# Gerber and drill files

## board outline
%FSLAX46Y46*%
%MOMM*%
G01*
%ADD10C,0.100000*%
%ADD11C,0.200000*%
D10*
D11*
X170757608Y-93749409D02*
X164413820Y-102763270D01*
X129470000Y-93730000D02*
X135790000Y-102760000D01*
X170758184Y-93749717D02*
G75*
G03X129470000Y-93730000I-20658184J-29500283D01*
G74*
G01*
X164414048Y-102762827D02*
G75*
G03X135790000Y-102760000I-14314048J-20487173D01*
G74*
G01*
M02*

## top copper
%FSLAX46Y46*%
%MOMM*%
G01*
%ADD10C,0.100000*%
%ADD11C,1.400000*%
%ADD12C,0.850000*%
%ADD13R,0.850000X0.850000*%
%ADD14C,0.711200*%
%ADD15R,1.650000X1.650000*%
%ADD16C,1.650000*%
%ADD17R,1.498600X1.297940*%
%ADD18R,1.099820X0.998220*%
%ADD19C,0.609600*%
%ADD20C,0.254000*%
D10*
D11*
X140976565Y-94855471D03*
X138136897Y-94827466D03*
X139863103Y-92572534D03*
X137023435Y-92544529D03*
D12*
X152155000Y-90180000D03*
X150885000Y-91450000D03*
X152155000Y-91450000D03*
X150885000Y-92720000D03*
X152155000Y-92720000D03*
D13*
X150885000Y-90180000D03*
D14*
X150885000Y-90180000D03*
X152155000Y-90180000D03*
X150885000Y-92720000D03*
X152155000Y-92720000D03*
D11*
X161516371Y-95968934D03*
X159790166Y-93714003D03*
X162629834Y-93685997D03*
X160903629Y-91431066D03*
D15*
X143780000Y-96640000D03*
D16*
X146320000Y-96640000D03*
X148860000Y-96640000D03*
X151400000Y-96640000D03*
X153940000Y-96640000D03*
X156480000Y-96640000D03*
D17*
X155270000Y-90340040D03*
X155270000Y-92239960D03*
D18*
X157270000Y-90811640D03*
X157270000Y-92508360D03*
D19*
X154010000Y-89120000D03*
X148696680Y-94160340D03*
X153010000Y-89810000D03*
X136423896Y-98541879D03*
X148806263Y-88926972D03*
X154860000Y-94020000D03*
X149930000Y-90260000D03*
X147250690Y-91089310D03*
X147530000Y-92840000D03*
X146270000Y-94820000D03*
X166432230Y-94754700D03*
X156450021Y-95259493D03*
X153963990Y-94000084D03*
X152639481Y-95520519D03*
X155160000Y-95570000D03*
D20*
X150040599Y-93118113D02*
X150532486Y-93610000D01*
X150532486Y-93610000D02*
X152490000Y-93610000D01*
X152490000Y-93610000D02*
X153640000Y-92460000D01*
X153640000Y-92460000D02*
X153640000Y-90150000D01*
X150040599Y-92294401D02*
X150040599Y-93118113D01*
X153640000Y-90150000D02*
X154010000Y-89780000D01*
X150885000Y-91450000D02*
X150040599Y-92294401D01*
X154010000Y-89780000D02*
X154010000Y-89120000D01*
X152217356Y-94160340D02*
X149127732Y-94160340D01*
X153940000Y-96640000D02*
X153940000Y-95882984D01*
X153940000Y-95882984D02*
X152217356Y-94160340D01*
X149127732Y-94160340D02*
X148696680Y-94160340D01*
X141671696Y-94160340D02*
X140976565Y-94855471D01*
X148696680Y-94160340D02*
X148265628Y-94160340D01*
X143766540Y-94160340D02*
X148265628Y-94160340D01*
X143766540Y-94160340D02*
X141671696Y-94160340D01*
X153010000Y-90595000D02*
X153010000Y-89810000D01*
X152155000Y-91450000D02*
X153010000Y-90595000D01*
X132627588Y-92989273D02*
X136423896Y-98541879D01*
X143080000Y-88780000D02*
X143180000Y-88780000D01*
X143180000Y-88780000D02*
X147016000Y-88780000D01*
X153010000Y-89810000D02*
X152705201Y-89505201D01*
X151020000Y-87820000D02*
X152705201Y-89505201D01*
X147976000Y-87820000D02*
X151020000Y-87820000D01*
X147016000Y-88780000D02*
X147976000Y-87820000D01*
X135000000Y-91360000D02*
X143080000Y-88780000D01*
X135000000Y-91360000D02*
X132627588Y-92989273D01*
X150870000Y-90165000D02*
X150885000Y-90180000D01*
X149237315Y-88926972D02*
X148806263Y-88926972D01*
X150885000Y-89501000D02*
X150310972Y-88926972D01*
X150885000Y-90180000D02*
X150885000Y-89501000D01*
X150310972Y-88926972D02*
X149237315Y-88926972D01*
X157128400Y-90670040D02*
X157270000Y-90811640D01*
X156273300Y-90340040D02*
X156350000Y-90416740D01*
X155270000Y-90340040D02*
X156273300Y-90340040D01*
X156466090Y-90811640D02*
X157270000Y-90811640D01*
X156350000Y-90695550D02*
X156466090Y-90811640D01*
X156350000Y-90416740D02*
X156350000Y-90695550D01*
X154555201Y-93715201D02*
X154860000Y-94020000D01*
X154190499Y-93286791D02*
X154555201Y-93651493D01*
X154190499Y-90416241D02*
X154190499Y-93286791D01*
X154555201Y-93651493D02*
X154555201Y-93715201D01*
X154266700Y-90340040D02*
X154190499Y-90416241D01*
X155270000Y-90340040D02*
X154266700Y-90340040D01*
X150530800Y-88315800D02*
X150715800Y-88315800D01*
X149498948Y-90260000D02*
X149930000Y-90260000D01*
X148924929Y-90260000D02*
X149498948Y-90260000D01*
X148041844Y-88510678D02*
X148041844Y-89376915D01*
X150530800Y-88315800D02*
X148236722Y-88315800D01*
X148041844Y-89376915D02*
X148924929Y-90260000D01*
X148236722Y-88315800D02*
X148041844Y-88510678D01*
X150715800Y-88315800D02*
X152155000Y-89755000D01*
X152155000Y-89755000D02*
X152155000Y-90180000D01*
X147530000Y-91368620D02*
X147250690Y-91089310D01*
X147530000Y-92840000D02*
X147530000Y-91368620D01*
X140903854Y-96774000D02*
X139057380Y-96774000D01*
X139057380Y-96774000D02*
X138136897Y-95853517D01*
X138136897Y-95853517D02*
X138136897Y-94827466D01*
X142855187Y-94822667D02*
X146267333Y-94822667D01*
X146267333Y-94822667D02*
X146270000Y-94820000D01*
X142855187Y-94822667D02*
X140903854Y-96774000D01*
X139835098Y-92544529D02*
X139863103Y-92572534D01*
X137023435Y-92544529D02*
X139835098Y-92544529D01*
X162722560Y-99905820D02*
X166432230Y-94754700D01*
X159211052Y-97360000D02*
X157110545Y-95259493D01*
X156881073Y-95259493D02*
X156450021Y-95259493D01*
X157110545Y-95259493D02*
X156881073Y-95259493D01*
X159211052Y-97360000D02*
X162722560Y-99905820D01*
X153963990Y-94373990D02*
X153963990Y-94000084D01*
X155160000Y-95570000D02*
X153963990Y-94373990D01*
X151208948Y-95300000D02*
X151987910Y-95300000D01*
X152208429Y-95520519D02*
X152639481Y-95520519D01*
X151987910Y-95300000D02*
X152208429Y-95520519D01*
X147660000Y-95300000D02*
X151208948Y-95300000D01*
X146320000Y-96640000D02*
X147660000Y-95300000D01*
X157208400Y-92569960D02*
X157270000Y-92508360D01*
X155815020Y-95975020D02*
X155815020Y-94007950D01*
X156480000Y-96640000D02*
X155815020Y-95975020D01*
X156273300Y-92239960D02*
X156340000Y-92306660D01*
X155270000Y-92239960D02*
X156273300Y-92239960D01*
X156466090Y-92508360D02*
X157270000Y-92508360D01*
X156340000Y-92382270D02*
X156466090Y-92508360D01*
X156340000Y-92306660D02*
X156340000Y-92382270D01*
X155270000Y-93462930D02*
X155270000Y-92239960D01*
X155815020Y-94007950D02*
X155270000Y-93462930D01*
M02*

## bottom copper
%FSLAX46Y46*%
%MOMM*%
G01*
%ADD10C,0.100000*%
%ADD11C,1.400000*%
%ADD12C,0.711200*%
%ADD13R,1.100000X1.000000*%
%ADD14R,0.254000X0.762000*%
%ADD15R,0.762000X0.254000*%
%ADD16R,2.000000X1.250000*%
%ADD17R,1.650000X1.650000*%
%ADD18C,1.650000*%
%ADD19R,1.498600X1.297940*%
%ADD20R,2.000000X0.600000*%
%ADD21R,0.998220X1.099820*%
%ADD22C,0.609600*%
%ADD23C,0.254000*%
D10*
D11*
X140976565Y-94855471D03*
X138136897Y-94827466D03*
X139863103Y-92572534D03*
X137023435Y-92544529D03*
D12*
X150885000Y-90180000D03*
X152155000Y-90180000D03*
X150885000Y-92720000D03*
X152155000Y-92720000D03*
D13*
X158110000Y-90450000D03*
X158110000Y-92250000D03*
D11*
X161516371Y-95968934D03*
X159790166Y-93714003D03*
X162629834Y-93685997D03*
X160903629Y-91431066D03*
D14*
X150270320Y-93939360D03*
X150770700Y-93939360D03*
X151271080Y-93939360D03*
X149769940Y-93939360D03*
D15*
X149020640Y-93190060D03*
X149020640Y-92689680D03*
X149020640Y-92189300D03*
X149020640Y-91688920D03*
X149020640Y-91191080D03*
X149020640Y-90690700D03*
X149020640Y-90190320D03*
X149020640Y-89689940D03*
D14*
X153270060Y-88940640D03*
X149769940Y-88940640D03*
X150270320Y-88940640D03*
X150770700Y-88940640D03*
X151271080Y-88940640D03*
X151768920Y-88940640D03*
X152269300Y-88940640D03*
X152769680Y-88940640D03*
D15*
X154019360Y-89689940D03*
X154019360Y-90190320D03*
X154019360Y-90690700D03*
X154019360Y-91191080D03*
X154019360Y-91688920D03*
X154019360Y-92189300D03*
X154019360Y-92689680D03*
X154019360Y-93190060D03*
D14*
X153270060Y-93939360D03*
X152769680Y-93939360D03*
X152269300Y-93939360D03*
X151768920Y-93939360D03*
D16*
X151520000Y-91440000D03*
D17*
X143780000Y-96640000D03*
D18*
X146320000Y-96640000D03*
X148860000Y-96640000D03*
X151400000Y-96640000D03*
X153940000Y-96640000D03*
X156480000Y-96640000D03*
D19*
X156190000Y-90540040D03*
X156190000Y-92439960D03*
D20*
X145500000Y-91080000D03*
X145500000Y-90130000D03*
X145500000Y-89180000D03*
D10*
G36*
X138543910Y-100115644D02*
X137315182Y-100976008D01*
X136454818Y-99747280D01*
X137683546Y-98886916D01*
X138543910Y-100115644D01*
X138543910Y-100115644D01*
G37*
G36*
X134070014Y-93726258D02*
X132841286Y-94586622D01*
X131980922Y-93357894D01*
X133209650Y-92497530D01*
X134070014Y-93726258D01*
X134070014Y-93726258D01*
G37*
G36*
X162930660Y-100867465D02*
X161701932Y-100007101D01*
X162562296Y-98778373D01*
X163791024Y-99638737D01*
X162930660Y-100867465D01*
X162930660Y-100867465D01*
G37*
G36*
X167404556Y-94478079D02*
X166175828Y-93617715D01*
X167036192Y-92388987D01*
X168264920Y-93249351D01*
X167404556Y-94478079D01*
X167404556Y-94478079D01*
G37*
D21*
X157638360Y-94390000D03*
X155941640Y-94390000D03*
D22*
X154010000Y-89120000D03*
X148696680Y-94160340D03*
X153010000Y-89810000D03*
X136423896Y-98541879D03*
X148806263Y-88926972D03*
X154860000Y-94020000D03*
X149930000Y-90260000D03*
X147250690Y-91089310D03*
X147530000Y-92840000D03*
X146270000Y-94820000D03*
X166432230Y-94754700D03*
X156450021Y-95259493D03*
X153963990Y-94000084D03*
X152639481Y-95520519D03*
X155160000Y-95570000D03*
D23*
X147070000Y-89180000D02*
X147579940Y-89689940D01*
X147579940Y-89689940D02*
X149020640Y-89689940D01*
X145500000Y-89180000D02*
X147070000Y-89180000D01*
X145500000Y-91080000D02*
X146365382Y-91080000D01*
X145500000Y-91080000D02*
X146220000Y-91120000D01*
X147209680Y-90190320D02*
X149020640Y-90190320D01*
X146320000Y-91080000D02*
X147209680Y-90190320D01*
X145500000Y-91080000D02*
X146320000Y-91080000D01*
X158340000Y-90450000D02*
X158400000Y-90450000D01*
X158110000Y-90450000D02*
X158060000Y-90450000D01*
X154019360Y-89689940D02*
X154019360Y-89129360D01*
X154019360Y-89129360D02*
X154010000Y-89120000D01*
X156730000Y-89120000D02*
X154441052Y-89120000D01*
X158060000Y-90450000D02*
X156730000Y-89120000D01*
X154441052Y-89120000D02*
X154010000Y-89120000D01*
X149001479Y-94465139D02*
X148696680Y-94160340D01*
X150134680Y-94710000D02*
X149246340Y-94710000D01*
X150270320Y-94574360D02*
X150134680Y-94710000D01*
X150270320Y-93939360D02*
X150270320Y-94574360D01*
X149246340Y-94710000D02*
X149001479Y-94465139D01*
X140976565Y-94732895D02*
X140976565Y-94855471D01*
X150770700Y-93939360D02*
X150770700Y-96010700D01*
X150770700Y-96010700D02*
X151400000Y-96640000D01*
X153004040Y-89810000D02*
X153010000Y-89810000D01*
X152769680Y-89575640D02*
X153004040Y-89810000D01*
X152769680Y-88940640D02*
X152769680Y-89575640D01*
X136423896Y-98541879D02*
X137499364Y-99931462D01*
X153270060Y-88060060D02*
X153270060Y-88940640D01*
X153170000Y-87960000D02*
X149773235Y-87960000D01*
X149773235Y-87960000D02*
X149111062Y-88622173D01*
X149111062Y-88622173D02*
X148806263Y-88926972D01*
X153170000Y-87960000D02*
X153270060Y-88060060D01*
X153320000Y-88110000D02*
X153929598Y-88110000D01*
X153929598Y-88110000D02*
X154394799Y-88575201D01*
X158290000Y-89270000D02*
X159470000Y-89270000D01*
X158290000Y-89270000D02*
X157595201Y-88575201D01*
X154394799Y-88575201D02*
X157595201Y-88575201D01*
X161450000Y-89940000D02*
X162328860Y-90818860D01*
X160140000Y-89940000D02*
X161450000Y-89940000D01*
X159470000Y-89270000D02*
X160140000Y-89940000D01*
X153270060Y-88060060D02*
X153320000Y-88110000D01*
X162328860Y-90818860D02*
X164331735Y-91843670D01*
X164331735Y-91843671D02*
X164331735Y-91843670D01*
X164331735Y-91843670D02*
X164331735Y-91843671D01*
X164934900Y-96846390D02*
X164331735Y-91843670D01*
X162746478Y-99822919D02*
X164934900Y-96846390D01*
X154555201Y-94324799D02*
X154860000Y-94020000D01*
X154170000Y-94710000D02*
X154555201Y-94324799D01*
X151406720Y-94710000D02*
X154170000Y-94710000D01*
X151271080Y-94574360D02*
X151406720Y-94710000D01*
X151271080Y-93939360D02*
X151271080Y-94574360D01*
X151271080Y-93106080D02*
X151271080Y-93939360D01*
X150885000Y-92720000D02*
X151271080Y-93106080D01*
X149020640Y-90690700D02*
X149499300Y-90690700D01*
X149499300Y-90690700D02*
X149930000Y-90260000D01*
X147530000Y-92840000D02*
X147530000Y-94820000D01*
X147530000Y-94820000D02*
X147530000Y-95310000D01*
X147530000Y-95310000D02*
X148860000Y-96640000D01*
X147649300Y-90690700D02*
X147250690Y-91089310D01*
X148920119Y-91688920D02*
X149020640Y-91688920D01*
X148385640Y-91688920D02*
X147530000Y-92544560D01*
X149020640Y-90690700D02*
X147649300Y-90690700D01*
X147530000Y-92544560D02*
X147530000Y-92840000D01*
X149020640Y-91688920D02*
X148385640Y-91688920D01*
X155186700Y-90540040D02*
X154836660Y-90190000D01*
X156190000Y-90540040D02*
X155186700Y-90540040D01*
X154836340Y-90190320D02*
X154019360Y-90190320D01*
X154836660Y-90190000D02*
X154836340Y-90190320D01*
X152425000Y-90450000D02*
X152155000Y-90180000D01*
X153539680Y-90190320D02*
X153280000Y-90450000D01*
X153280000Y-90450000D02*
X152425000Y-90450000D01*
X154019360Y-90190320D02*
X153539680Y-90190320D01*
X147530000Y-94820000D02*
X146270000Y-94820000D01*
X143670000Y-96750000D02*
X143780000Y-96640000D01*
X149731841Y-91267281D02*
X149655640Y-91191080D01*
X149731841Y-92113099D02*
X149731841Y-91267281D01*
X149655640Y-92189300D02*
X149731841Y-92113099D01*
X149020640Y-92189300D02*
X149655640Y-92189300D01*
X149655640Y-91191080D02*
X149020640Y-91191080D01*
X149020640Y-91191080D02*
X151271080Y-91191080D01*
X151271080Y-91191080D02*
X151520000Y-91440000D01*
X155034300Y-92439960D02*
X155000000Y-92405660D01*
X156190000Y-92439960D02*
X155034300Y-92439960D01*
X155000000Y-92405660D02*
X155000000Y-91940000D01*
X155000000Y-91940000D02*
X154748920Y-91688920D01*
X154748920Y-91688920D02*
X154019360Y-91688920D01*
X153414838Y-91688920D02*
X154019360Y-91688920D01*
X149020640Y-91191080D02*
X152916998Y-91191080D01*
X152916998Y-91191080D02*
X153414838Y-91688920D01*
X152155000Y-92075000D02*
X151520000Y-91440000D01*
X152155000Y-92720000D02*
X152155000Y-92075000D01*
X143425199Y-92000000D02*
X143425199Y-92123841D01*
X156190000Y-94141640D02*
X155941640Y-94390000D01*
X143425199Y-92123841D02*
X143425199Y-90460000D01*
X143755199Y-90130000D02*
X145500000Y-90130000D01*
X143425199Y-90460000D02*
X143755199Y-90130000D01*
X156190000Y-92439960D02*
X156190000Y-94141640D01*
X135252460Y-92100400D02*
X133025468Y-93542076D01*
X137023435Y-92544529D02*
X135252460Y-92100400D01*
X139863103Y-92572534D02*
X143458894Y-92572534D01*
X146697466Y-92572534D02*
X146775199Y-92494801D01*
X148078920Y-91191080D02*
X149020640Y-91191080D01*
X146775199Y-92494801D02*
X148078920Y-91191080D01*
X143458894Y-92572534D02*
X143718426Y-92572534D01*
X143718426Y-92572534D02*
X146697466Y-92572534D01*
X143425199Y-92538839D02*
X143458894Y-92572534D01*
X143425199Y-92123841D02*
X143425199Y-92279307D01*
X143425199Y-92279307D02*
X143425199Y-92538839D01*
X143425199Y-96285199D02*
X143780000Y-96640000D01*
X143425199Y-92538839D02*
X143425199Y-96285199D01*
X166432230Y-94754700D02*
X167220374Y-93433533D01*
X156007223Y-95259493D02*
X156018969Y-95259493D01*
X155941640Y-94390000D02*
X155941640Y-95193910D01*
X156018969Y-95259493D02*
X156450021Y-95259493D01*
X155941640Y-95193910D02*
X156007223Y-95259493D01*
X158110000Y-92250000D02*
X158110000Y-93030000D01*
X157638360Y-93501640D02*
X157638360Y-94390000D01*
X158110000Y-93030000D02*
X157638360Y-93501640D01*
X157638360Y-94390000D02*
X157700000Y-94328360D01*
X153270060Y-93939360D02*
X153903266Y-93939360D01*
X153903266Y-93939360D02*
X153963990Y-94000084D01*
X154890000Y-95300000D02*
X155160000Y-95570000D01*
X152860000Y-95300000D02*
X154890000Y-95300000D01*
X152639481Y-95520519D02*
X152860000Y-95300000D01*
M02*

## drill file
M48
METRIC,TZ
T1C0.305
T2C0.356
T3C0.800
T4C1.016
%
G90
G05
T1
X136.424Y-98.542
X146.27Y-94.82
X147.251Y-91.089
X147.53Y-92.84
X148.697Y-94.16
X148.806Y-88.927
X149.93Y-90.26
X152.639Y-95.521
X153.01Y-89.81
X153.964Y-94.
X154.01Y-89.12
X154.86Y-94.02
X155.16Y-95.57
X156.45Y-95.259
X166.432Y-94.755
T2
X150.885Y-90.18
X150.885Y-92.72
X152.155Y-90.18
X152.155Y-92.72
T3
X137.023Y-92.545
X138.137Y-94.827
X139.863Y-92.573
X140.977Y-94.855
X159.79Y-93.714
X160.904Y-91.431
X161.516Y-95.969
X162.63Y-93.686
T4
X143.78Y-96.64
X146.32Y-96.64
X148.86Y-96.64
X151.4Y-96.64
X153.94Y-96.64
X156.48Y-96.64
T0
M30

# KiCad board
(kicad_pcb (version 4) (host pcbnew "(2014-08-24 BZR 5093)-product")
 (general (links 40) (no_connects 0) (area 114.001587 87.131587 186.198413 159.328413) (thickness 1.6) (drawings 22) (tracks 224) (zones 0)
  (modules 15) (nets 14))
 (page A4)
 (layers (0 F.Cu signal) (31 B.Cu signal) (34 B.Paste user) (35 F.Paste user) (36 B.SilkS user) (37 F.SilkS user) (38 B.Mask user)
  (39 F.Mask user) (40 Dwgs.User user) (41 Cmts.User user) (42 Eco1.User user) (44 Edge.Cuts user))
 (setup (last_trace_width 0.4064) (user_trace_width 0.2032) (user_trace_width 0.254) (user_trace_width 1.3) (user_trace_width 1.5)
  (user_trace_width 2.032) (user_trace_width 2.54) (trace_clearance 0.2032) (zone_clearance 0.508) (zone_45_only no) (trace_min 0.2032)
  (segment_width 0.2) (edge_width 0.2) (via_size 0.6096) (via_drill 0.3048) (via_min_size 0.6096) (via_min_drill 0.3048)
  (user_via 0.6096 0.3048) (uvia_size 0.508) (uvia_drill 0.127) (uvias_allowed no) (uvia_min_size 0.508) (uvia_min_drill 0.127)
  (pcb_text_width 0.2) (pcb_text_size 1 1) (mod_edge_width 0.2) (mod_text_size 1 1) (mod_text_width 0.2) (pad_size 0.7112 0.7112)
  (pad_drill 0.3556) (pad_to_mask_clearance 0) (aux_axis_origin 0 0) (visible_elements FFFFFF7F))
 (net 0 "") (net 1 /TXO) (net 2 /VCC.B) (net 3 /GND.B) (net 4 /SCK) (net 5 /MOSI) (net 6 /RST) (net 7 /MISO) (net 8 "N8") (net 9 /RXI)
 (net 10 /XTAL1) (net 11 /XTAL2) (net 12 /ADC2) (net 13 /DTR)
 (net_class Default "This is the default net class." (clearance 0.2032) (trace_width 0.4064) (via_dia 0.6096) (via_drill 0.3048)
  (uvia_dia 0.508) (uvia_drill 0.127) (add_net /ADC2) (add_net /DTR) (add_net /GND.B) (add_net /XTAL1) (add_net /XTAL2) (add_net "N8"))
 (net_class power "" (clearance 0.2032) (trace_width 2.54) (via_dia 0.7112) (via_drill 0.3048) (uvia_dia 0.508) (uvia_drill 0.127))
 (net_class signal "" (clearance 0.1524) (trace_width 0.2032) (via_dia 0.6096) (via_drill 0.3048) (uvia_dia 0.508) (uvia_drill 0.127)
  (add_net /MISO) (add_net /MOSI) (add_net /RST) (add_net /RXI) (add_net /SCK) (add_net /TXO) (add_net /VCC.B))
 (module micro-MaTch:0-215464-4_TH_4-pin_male (layer F.Cu) (at 139 93.7 296)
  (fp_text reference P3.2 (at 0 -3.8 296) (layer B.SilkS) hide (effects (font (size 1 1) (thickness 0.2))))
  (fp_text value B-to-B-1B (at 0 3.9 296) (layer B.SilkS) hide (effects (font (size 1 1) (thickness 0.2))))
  (pad 1 thru_hole circle (at 1.905 -1.27 296) (size 1.4 1.4) (drill 0.8) (layers *.Cu *.Mask) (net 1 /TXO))
  (pad 2 thru_hole circle (at 0.635 1.27 296) (size 1.4 1.4) (drill 0.8) (layers *.Cu *.Mask) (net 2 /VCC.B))
  (pad 3 thru_hole circle (at -0.635 -1.27 296) (size 1.4 1.4) (drill 0.8) (layers *.Cu *.Mask) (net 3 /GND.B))
  (pad 4 thru_hole circle (at -1.905 1.27 296) (size 1.4 1.4) (drill 0.8) (layers *.Cu *.Mask) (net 3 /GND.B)))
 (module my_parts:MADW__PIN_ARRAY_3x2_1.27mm (layer F.Cu) (at 151.52 91.45 270) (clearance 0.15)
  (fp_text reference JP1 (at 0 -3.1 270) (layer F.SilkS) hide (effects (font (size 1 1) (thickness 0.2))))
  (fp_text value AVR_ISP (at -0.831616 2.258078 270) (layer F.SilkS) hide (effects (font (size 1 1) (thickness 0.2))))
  (pad 2 smd circle (at -1.27 -0.635 270) (size 0.85 0.85) (layers F.Cu F.Mask) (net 2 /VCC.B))
  (pad 3 smd circle (at 0 0.635 270) (size 0.85 0.85) (layers F.Cu F.Mask) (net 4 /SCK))
  (pad 4 smd circle (at 0 -0.635 270) (size 0.85 0.85) (layers F.Cu F.Mask) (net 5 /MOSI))
  (pad 5 smd circle (at 1.27 0.635 270) (size 0.85 0.85) (layers F.Cu F.Mask) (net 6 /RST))
  (pad 6 smd circle (at 1.27 -0.635 270) (size 0.85 0.85) (layers F.Cu F.Mask) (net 3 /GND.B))
  (pad 1 smd rect (at -1.27 0.635 270) (size 0.85 0.85) (layers F.Cu F.Mask) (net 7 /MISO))
  (pad 1 thru_hole circle (at -1.27 0.635 270) (size 0.7112 0.7112) (drill 0.3556) (layers *.Cu F.Mask) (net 7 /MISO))
  (pad 2 thru_hole circle (at -1.27 -0.635 270) (size 0.7112 0.7112) (drill 0.3556) (layers *.Cu F.Mask) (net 2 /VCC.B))
  (pad 5 thru_hole circle (at 1.27 0.635 270) (size 0.7112 0.7112) (drill 0.3556) (layers *.Cu F.Mask) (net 6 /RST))
  (pad 6 thru_hole circle (at 1.27 -0.635 270) (size 0.7112 0.7112) (drill 0.3556) (layers *.Cu F.Mask) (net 3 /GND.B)))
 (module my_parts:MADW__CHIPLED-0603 (layer B.Cu) (at 158.11 91.35 270)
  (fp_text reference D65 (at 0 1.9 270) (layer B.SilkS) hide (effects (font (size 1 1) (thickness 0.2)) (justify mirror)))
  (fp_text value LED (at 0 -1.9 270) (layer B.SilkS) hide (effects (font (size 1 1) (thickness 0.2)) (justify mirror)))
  (pad 1 smd rect (at -0.9 0 270) (size 1 1.1) (layers B.Cu B.Paste B.Mask) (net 4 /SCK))
  (pad 2 smd rect (at 0.9 0 270) (size 1 1.1) (layers B.Cu B.Paste B.Mask) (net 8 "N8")))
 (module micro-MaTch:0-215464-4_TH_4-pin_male (layer F.Cu) (at 161.21 93.7 244)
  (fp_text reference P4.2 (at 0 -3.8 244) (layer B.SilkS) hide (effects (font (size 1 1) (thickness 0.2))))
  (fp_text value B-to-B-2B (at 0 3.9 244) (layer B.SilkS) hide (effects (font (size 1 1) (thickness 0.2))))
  (pad 1 thru_hole circle (at 1.905 -1.27 244) (size 1.4 1.4) (drill 0.8) (layers *.Cu *.Mask))
  (pad 2 thru_hole circle (at 0.635 1.27 244) (size 1.4 1.4) (drill 0.8) (layers *.Cu *.Mask))
  (pad 3 thru_hole circle (at -0.635 -1.27 244) (size 1.4 1.4) (drill 0.8) (layers *.Cu *.Mask))
  (pad 4 thru_hole circle (at -1.905 1.27 244) (size 1.4 1.4) (drill 0.8) (layers *.Cu *.Mask)))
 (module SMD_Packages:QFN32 (layer B.Cu) (at 151.52 91.44)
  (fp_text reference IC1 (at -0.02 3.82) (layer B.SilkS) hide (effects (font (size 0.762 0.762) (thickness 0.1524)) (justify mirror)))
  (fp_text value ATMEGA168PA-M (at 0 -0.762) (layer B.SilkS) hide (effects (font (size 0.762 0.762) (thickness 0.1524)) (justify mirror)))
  (pad 31 smd rect (at -1.24968 2.49936) (size 0.254 0.762) (layers B.Cu B.Paste B.Mask) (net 1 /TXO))
  (pad 30 smd rect (at -0.7493 2.49936) (size 0.254 0.762) (layers B.Cu B.Paste B.Mask) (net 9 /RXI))
  (pad 29 smd rect (at -0.24892 2.49936) (size 0.254 0.762) (layers B.Cu B.Paste B.Mask) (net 6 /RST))
  (pad 32 smd rect (at -1.75006 2.49936) (size 0.254 0.762) (layers B.Cu B.Paste B.Mask))
  (pad 1 smd rect (at -2.49936 1.75006 270) (size 0.254 0.762) (layers B.Cu B.Paste B.Mask))
  (pad 2 smd rect (at -2.49936 1.24968 270) (size 0.254 0.762) (layers B.Cu B.Paste B.Mask))
  (pad 3 smd rect (at -2.49936 0.7493 270) (size 0.254 0.762) (layers B.Cu B.Paste B.Mask) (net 3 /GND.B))
  (pad 4 smd rect (at -2.49936 0.24892 270) (size 0.254 0.762) (layers B.Cu B.Paste B.Mask) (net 2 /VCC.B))
  (pad 5 smd rect (at -2.49936 -0.24892 270) (size 0.254 0.762) (layers B.Cu B.Paste B.Mask) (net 3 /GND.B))
  (pad 6 smd rect (at -2.49936 -0.7493 270) (size 0.254 0.762) (layers B.Cu B.Paste B.Mask) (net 2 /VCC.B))
  (pad 7 smd rect (at -2.49936 -1.24968 270) (size 0.254 0.762) (layers B.Cu B.Paste B.Mask) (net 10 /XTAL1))
  (pad 8 smd rect (at -2.49936 -1.75006 270) (size 0.254 0.762) (layers B.Cu B.Paste B.Mask) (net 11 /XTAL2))
  (pad 16 smd rect (at 1.75006 -2.49936) (size 0.254 0.762) (layers B.Cu B.Paste B.Mask) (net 7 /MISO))
  (pad 9 smd rect (at -1.75006 -2.49936) (size 0.254 0.762) (layers B.Cu B.Paste B.Mask))
  (pad 10 smd rect (at -1.24968 -2.49936) (size 0.254 0.762) (layers B.Cu B.Paste B.Mask))
  (pad 11 smd rect (at -0.7493 -2.49936) (size 0.254 0.762) (layers B.Cu B.Paste B.Mask))
  (pad 12 smd rect (at -0.24892 -2.49936) (size 0.254 0.762) (layers B.Cu B.Paste B.Mask))
  (pad 13 smd rect (at 0.24892 -2.49936) (size 0.254 0.762) (layers B.Cu B.Paste B.Mask))
  (pad 14 smd rect (at 0.7493 -2.49936) (size 0.254 0.762) (layers B.Cu B.Paste B.Mask))
  (pad 15 smd rect (at 1.24968 -2.49936) (size 0.254 0.762) (layers B.Cu B.Paste B.Mask) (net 5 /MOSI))
  (pad 17 smd rect (at 2.49936 -1.75006 270) (size 0.254 0.762) (layers B.Cu B.Paste B.Mask) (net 4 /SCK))
  (pad 18 smd rect (at 2.49936 -1.24968 270) (size 0.254 0.762) (layers B.Cu B.Paste B.Mask) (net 2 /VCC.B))
  (pad 19 smd rect (at 2.49936 -0.7493 270) (size 0.254 0.762) (layers B.Cu B.Paste B.Mask))
  (pad 20 smd rect (at 2.49936 -0.24892 270) (size 0.254 0.762) (layers B.Cu B.Paste B.Mask))
  (pad 21 smd rect (at 2.49936 0.24892 270) (size 0.254 0.762) (layers B.Cu B.Paste B.Mask) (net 3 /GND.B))
  (pad 22 smd rect (at 2.49936 0.7493 270) (size 0.254 0.762) (layers B.Cu B.Paste B.Mask))
  (pad 23 smd rect (at 2.49936 1.24968 270) (size 0.254 0.762) (layers B.Cu B.Paste B.Mask))
  (pad 24 smd rect (at 2.49936 1.75006 270) (size 0.254 0.762) (layers B.Cu B.Paste B.Mask))
  (pad 25 smd rect (at 1.75006 2.49936) (size 0.254 0.762) (layers B.Cu B.Paste B.Mask) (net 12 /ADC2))
  (pad 26 smd rect (at 1.24968 2.49936) (size 0.254 0.762) (layers B.Cu B.Paste B.Mask))
  (pad 27 smd rect (at 0.7493 2.49936) (size 0.254 0.762) (layers B.Cu B.Paste B.Mask))
  (pad 28 smd rect (at 0.24892 2.49936) (size 0.254 0.762) (layers B.Cu B.Paste B.Mask))
  (pad 33 smd rect (at 0 0) (size 2 1.25) (layers B.Cu B.Paste B.Mask) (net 3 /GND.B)))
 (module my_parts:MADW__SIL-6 (layer B.Cu) (at 150.13 96.64)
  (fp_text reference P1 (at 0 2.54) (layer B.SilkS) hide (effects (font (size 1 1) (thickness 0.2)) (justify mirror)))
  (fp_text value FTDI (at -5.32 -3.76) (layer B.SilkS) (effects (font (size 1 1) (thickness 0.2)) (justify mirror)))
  (pad 1 thru_hole rect (at -6.35 0) (size 1.65 1.65) (drill 1.016) (layers *.Cu *.Mask B.SilkS) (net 3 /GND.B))
  (pad 2 thru_hole circle (at -3.81 0) (size 1.65 1.65) (drill 1.016) (layers *.Cu *.Mask B.SilkS) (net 12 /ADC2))
  (pad 3 thru_hole circle (at -1.27 0) (size 1.65 1.65) (drill 1.016) (layers *.Cu *.Mask B.SilkS) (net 2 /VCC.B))
  (pad 4 thru_hole circle (at 1.27 0) (size 1.65 1.65) (drill 1.016) (layers *.Cu *.Mask B.SilkS) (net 9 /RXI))
  (pad 5 thru_hole circle (at 3.81 0) (size 1.65 1.65) (drill 1.016) (layers *.Cu *.Mask B.SilkS) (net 1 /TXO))
  (pad 6 thru_hole circle (at 6.35 0) (size 1.65 1.65) (drill 1.016) (layers *.Cu *.Mask B.SilkS) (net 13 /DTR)))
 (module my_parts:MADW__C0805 (layer B.Cu) (at 156.19 91.49 270)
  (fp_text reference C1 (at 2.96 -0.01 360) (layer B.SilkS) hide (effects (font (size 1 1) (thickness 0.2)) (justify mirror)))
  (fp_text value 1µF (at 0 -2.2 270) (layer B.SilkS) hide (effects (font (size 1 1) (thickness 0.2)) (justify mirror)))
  (pad 1 smd rect (at -0.94996 0 270) (size 1.29794 1.4986) (layers B.Cu B.Paste B.Mask) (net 2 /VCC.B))
  (pad 2 smd rect (at 0.94996 0 270) (size 1.29794 1.4986) (layers B.Cu B.Paste B.Mask) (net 3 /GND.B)))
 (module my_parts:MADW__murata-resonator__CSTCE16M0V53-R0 (layer B.Cu) (at 145.5 90.13 90)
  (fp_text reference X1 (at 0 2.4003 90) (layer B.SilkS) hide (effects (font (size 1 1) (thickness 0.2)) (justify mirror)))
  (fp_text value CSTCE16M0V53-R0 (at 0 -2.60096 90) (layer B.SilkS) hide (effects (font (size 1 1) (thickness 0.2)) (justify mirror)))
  (pad 1 smd rect (at -0.95 0 90) (size 0.6 2) (layers B.Cu B.Paste B.Mask) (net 10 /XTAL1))
  (pad 2 smd rect (at 0 0 90) (size 0.6 2) (layers B.Cu B.Paste B.Mask) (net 3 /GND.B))
  (pad 3 smd rect (at 0.95 0 90) (size 0.6 2) (layers B.Cu B.Paste B.Mask) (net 11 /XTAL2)))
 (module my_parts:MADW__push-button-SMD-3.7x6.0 (layer B.Cu) (at 135.262416 96.736769 125)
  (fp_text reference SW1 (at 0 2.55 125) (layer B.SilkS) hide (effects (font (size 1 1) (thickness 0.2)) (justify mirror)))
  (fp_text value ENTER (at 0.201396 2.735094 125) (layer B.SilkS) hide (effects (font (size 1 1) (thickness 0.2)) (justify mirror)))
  (pad 1 smd rect (at -3.9 0 125) (size 1.5 1.5) (layers B.Cu B.Paste B.Mask) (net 5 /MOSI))
  (pad 2 smd rect (at 3.9 0 125) (size 1.5 1.5) (layers B.Cu B.Paste B.Mask) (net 3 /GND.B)))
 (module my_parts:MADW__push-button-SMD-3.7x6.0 (layer B.Cu) (at 164.983426 96.628226 55)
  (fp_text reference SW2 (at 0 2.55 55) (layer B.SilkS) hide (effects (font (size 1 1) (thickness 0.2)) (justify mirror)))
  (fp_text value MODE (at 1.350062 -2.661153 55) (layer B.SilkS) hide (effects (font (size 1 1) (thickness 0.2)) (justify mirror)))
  (pad 1 smd rect (at -3.9 0 55) (size 1.5 1.5) (layers B.Cu B.Paste B.Mask) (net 7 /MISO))
  (pad 2 smd rect (at 3.9 0 55) (size 1.5 1.5) (layers B.Cu B.Paste B.Mask) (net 3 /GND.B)))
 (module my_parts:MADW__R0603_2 (layer B.Cu) (at 156.79 94.39 180)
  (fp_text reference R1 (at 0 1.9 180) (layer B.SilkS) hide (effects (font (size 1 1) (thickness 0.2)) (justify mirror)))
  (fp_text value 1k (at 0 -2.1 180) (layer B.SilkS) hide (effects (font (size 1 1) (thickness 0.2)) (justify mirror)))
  (pad 1 smd rect (at -0.84836 0 180) (size 0.99822 1.09982) (layers B.Cu B.Paste B.Mask) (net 8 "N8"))
  (pad 2 smd rect (at 0.84836 0 180) (size 0.99822 1.09982) (layers B.Cu B.Paste B.Mask) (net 3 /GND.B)))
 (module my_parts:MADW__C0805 (layer F.Cu) (at 155.27 91.29 270)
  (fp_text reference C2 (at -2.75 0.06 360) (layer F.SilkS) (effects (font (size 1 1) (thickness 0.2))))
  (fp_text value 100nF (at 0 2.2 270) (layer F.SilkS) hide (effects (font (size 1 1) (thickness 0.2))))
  (pad 1 smd rect (at -0.94996 0 270) (size 1.29794 1.4986) (layers F.Cu F.Paste F.Mask) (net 6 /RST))
  (pad 2 smd rect (at 0.94996 0 270) (size 1.29794 1.4986) (layers F.Cu F.Paste F.Mask) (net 13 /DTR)))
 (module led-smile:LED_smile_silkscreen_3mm (layer B.Cu) (at 141.65 90.42)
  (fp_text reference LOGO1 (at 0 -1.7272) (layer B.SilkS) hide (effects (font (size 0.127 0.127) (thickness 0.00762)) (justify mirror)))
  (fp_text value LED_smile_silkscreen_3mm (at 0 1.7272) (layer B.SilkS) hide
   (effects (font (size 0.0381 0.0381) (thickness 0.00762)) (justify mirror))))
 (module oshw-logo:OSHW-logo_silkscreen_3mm (layer F.Cu) (at 144.59 91.96)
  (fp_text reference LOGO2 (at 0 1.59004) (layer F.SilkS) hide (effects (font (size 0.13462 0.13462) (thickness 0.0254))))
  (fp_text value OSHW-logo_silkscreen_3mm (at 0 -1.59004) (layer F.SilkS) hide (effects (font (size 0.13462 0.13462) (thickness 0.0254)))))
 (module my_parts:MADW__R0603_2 (layer F.Cu) (at 157.27 91.66 270)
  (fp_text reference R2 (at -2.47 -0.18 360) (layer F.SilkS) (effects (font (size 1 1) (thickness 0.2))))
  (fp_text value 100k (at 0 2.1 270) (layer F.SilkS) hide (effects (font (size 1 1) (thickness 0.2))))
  (pad 1 smd rect (at -0.84836 0 270) (size 0.99822 1.09982) (layers F.Cu F.Paste F.Mask) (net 6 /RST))
  (pad 2 smd rect (at 0.84836 0 270) (size 0.99822 1.09982) (layers F.Cu F.Paste F.Mask) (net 13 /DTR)))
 (gr_line (start 170.757608 93.749409) (end 164.41382 102.76327) (layer Edge.Cuts) (width 0.2))
 (gr_line (start 129.47 93.73) (end 135.79 102.76) (layer Edge.Cuts) (width 0.2))
 (gr_arc (start 150.1 123.25) (end 129.47 93.73) (angle 69.95013535) (layer Edge.Cuts) (width 0.2))
 (gr_arc (start 150.1 123.25) (end 135.79 102.76) (angle 69.87140367) (layer Edge.Cuts) (width 0.2))
 (segment (start 147.07 89.18) (end 147.57994 89.68994) (width 0.254) (layer B.Cu) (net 11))
 (segment (start 147.57994 89.68994) (end 149.02064 89.68994) (width 0.254) (layer B.Cu) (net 11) (status 20))
 (segment (start 145.5 89.18) (end 147.07 89.18) (width 0.254) (layer B.Cu) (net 11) (status 10))
 (segment (start 145.5 91.08) (end 146.365382 91.08) (width 0.254) (layer B.Cu) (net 10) (status 30))
 (segment (start 145.5 91.08) (end 146.22 91.12) (width 0.254) (layer B.Cu) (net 10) (status 30))
 (segment (start 147.20968 90.19032) (end 149.02064 90.19032) (width 0.254) (layer B.Cu) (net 10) (status 20))
 (segment (start 146.32 91.08) (end 147.20968 90.19032) (width 0.254) (layer B.Cu) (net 10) (status 10))
 (segment (start 145.5 91.08) (end 146.32 91.08) (width 0.254) (layer B.Cu) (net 10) (status 30))
 (segment (start 150.040599 93.118113) (end 150.532486 93.61) (width 0.254) (layer F.Cu) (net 4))
 (segment (start 150.532486 93.61) (end 152.49 93.61) (width 0.254) (layer F.Cu) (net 4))
 (segment (start 152.49 93.61) (end 153.64 92.46) (width 0.254) (layer F.Cu) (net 4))
 (segment (start 153.64 92.46) (end 153.64 90.15) (width 0.254) (layer F.Cu) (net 4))
 (segment (start 150.040599 92.294401) (end 150.040599 93.118113) (width 0.254) (layer F.Cu) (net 4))
 (segment (start 153.64 90.15) (end 154.01 89.78) (width 0.254) (layer F.Cu) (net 4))
 (segment (start 150.885 91.45) (end 150.040599 92.294401) (width 0.254) (layer F.Cu) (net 4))
 (segment (start 154.01 89.78) (end 154.01 89.12) (width 0.254) (layer F.Cu) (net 4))
 (segment (start 158.34 90.45) (end 158.4 90.45) (width 0.254) (layer B.Cu) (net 4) (status 30))
 (via (at 154.01 89.12) (size 0.6096) (drill 0.3048) (layers F.Cu B.Cu) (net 4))
 (segment (start 158.11 90.45) (end 158.06 90.45) (width 0.254) (layer B.Cu) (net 4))
 (segment (start 154.01936 89.68994) (end 154.01936 89.12936) (width 0.254) (layer B.Cu) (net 4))
 (segment (start 154.01936 89.12936) (end 154.01 89.12) (width 0.254) (layer B.Cu) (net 4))
 (segment (start 156.73 89.12) (end 154.441052 89.12) (width 0.254) (layer B.Cu) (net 4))
 (segment (start 158.06 90.45) (end 156.73 89.12) (width 0.254) (layer B.Cu) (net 4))
 (segment (start 154.441052 89.12) (end 154.01 89.12) (width 0.254) (layer B.Cu) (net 4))
 (segment (start 152.217356 94.16034) (end 149.127732 94.16034) (width 0.254) (layer F.Cu) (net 1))
 (segment (start 153.94 96.64) (end 153.94 95.882984) (width 0.254) (layer F.Cu) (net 1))
 (segment (start 153.94 95.882984) (end 152.217356 94.16034) (width 0.254) (layer F.Cu) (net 1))
 (segment (start 149.001479 94.465139) (end 148.69668 94.16034) (width 0.254) (layer B.Cu) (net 1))
 (segment (start 149.127732 94.16034) (end 148.69668 94.16034) (width 0.254) (layer F.Cu) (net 1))
 (segment (start 150.13468 94.71) (end 149.24634 94.71) (width 0.254) (layer B.Cu) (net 1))
 (segment (start 150.27032 94.57436) (end 150.13468 94.71) (width 0.254) (layer B.Cu) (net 1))
 (segment (start 150.27032 93.93936) (end 150.27032 94.57436) (width 0.254) (layer B.Cu) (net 1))
 (via (at 148.69668 94.16034) (size 0.6096) (drill 0.3048) (layers F.Cu B.Cu) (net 1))
 (segment (start 149.24634 94.71) (end 149.001479 94.465139) (width 0.254) (layer B.Cu) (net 1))
 (segment (start 140.976565 94.732895) (end 140.976565 94.855471) (width 0.254) (layer B.Cu) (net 1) (status 30))
 (segment (start 141.671696 94.16034) (end 140.976565 94.855471) (width 0.254) (layer F.Cu) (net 1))
 (segment (start 148.69668 94.16034) (end 148.265628 94.16034) (width 0.254) (layer F.Cu) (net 1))
 (segment (start 143.76654 94.16034) (end 148.265628 94.16034) (width 0.254) (layer F.Cu) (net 1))
 (segment (start 143.76654 94.16034) (end 141.671696 94.16034) (width 0.254) (layer F.Cu) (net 1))
 (segment (start 150.7707 93.93936) (end 150.7707 96.0107) (width 0.254) (layer B.Cu) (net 9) (status 10))
 (segment (start 150.7707 96.0107) (end 151.4 96.64) (width 0.254) (layer B.Cu) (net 9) (status 20))
 (via (at 153.01 89.81) (size 0.6096) (drill 0.3048) (layers F.Cu B.Cu) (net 5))
 (segment (start 153.00404 89.81) (end 153.01 89.81) (width 0.254) (layer B.Cu) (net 5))
 (segment (start 152.76968 89.57564) (end 153.00404 89.81) (width 0.254) (layer B.Cu) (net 5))
 (segment (start 152.76968 88.94064) (end 152.76968 89.57564) (width 0.254) (layer B.Cu) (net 5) (status 10))
 (segment (start 153.01 90.595) (end 153.01 89.81) (width 0.254) (layer F.Cu) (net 5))
 (segment (start 152.155 91.45) (end 153.01 90.595) (width 0.254) (layer F.Cu) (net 5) (status 10))
 (segment (start 132.627588 92.989273) (end 136.423896 98.541879) (width 0.254) (layer F.Cu) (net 5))
 (via (at 136.423896 98.541879) (size 0.6096) (layers F.Cu B.Cu) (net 5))
 (segment (start 136.423896 98.541879) (end 137.499364 99.931462) (width 0.254) (layer B.Cu) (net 5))
 (segment (start 143.08 88.78) (end 143.18 88.78) (width 0.254) (layer F.Cu) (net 5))
 (segment (start 143.18 88.78) (end 147.016 88.78) (width 0.254) (layer F.Cu) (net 5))
 (segment (start 153.01 89.81) (end 152.705201 89.505201) (width 0.254) (layer F.Cu) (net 5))
 (segment (start 151.02 87.82) (end 152.705201 89.505201) (width 0.254) (layer F.Cu) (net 5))
 (segment (start 147.976 87.82) (end 151.02 87.82) (width 0.254) (layer F.Cu) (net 5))
 (segment (start 147.016 88.78) (end 147.976 87.82) (width 0.254) (layer F.Cu) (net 5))
 (segment (start 135 91.36) (end 143.08 88.78) (width 0.254) (layer F.Cu) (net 5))
 (segment (start 135 91.36) (end 132.627588 92.989273) (width 0.254) (layer F.Cu) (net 5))
 (segment (start 150.87 90.165) (end 150.885 90.18) (width 0.254) (layer F.Cu) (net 7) (status 30))
 (segment (start 153.27006 88.06006) (end 153.27006 88.94064) (width 0.254) (layer B.Cu) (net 7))
 (via (at 148.806263 88.926972) (size 0.6096) (drill 0.3048) (layers F.Cu B.Cu) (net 7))
 (segment (start 153.17 87.96) (end 149.773235 87.96) (width 0.254) (layer B.Cu) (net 7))
 (segment (start 149.773235 87.96) (end 149.111062 88.622173) (width 0.254) (layer B.Cu) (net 7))
 (segment (start 149.237315 88.926972) (end 148.806263 88.926972) (width 0.254) (layer F.Cu) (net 7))
 (segment (start 150.885 89.501) (end 150.310972 88.926972) (width 0.254) (layer F.Cu) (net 7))
 (segment (start 149.111062 88.622173) (end 148.806263 88.926972) (width 0.254) (layer B.Cu) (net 7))
 (segment (start 150.885 90.18) (end 150.885 89.501) (width 0.254) (layer F.Cu) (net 7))
 (segment (start 150.310972 88.926972) (end 149.237315 88.926972) (width 0.254) (layer F.Cu) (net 7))
 (segment (start 153.17 87.96) (end 153.27006 88.06006) (width 0.254) (layer B.Cu) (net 7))
 (segment (start 153.32 88.11) (end 153.929598 88.11) (width 0.254) (layer B.Cu) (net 7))
 (segment (start 153.929598 88.11) (end 154.394799 88.575201) (width 0.254) (layer B.Cu) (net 7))
 (segment (start 158.29 89.27) (end 159.47 89.27) (width 0.254) (layer B.Cu) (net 7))
 (segment (start 158.29 89.27) (end 157.595201 88.575201) (width 0.254) (layer B.Cu) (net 7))
 (segment (start 154.394799 88.575201) (end 157.595201 88.575201) (width 0.254) (layer B.Cu) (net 7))
 (segment (start 161.45 89.94) (end 162.32886 90.81886) (width 0.254) (layer B.Cu) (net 7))
 (segment (start 160.14 89.94) (end 161.45 89.94) (width 0.254) (layer B.Cu) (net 7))
 (segment (start 159.47 89.27) (end 160.14 89.94) (width 0.254) (layer B.Cu) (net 7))
 (segment (start 153.27006 88.06006) (end 153.32 88.11) (width 0.254) (layer B.Cu) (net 7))
 (segment (start 162.32886 90.81886) (end 164.331735 91.84367) (width 0.254) (layer B.Cu) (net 7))
 (segment (start 164.331735 91.843671) (end 164.331735 91.84367) (width 0.254) (layer B.Cu) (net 7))
 (segment (start 164.331735 91.84367) (end 164.331735 91.843671) (width 0.254) (layer B.Cu) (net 7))
 (segment (start 164.9349 96.84639) (end 164.331735 91.84367) (width 0.254) (layer B.Cu) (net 7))
 (segment (start 162.746478 99.822919) (end 164.9349 96.84639) (width 0.254) (layer B.Cu) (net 7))
 (segment (start 154.555201 94.324799) (end 154.86 94.02) (width 0.254) (layer B.Cu) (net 6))
 (segment (start 154.17 94.71) (end 154.555201 94.324799) (width 0.254) (layer B.Cu) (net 6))
 (segment (start 151.40672 94.71) (end 154.17 94.71) (width 0.254) (layer B.Cu) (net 6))
 (segment (start 151.27108 94.57436) (end 151.40672 94.71) (width 0.254) (layer B.Cu) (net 6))
 (segment (start 151.27108 93.93936) (end 151.27108 94.57436) (width 0.254) (layer B.Cu) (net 6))
 (via (at 154.86 94.02) (size 0.6096) (drill 0.3048) (layers F.Cu B.Cu) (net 6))
 (segment (start 151.27108 93.10608) (end 151.27108 93.93936) (width 0.254) (layer B.Cu) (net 6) (status 20))
 (segment (start 150.885 92.72) (end 151.27108 93.10608) (width 0.254) (layer B.Cu) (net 6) (status 10))
 (segment (start 157.1284 90.67004) (end 157.27 90.81164) (width 0.254) (layer F.Cu) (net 6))
 (segment (start 156.2733 90.34004) (end 156.35 90.41674) (width 0.254) (layer F.Cu) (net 6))
 (segment (start 155.27 90.34004) (end 156.2733 90.34004) (width 0.254) (layer F.Cu) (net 6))
 (segment (start 156.46609 90.81164) (end 157.27 90.81164) (width 0.254) (layer F.Cu) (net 6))
 (segment (start 156.35 90.69555) (end 156.46609 90.81164) (width 0.254) (layer F.Cu) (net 6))
 (segment (start 156.35 90.41674) (end 156.35 90.69555) (width 0.254) (layer F.Cu) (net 6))
 (segment (start 154.555201 93.715201) (end 154.86 94.02) (width 0.254) (layer F.Cu) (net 6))
 (segment (start 154.190499 93.286791) (end 154.555201 93.651493) (width 0.254) (layer F.Cu) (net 6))
 (segment (start 154.190499 90.416241) (end 154.190499 93.286791) (width 0.254) (layer F.Cu) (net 6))
 (segment (start 154.555201 93.651493) (end 154.555201 93.715201) (width 0.254) (layer F.Cu) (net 6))
 (segment (start 154.2667 90.34004) (end 154.190499 90.416241) (width 0.254) (layer F.Cu) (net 6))
 (segment (start 155.27 90.34004) (end 154.2667 90.34004) (width 0.254) (layer F.Cu) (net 6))
 (segment (start 150.5308 88.3158) (end 150.7158 88.3158) (width 0.254) (layer F.Cu) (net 2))
 (segment (start 149.02064 90.6907) (end 149.4993 90.6907) (width 0.254) (layer B.Cu) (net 2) (status 10))
 (segment (start 149.4993 90.6907) (end 149.93 90.26) (width 0.254) (layer B.Cu) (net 2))
 (via (at 149.93 90.26) (size 0.6096) (drill 0.3048) (layers F.Cu B.Cu) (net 2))
 (segment (start 149.498948 90.26) (end 149.93 90.26) (width 0.254) (layer F.Cu) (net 2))
 (segment (start 148.924929 90.26) (end 149.498948 90.26) (width 0.254) (layer F.Cu) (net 2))
 (segment (start 148.041844 88.510678) (end 148.041844 89.376915) (width 0.254) (layer F.Cu) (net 2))
 (segment (start 150.5308 88.3158) (end 148.236722 88.3158) (width 0.254) (layer F.Cu) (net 2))
 (segment (start 148.041844 89.376915) (end 148.924929 90.26) (width 0.254) (layer F.Cu) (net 2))
 (segment (start 148.236722 88.3158) (end 148.041844 88.510678) (width 0.254) (layer F.Cu) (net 2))
 (segment (start 150.7158 88.3158) (end 152.155 89.755) (width 0.254) (layer F.Cu) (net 2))
 (segment (start 152.155 89.755) (end 152.155 90.18) (width 0.254) (layer F.Cu) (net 2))
 (segment (start 147.53 92.84) (end 147.53 94.82) (width 0.254) (layer B.Cu) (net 2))
 (segment (start 147.53 94.82) (end 147.53 95.31) (width 0.254) (layer B.Cu) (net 2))
 (segment (start 147.53 95.31) (end 148.86 96.64) (width 0.254) (layer B.Cu) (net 2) (status 20))
 (segment (start 147.6493 90.6907) (end 147.25069 91.08931) (width 0.254) (layer B.Cu) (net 2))
 (segment (start 147.53 91.36862) (end 147.25069 91.08931) (width 0.254) (layer F.Cu) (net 2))
 (segment (start 147.53 92.84) (end 147.53 91.36862) (width 0.254) (layer F.Cu) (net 2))
 (segment (start 148.920119 91.68892) (end 149.02064 91.68892) (width 0.254) (layer B.Cu) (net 2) (status 30))
 (segment (start 148.38564 91.68892) (end 147.53 92.54456) (width 0.254) (layer B.Cu) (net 2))
 (segment (start 149.02064 90.6907) (end 147.6493 90.6907) (width 0.254) (layer B.Cu) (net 2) (status 10))
 (segment (start 147.53 92.54456) (end 147.53 92.84) (width 0.254) (layer B.Cu) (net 2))
 (segment (start 149.02064 91.68892) (end 148.38564 91.68892) (width 0.254) (layer B.Cu) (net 2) (status 10))
 (via (at 147.25069 91.08931) (size 0.6096) (drill 0.3048) (layers F.Cu B.Cu) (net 2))
 (via (at 147.53 92.84) (size 0.6096) (drill 0.3048) (layers F.Cu B.Cu) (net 2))
 (segment (start 155.1867 90.54004) (end 154.83666 90.19) (width 0.254) (layer B.Cu) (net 2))
 (segment (start 156.19 90.54004) (end 155.1867 90.54004) (width 0.254) (layer B.Cu) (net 2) (status 10))
 (segment (start 154.83634 90.19032) (end 154.01936 90.19032) (width 0.254) (layer B.Cu) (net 2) (status 20))
 (segment (start 154.83666 90.19) (end 154.83634 90.19032) (width 0.254) (layer B.Cu) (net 2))
 (segment (start 152.425 90.45) (end 152.155 90.18) (width 0.254) (layer B.Cu) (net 2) (status 30))
 (segment (start 153.53968 90.19032) (end 153.28 90.45) (width 0.254) (layer B.Cu) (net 2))
 (segment (start 153.28 90.45) (end 152.425 90.45) (width 0.254) (layer B.Cu) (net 2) (status 20))
 (segment (start 154.01936 90.19032) (end 153.53968 90.19032) (width 0.254) (layer B.Cu) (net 2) (status 10))
 (segment (start 140.903854 96.774) (end 139.05738 96.774) (width 0.254) (layer F.Cu) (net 2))
 (segment (start 139.05738 96.774) (end 138.136897 95.853517) (width 0.254) (layer F.Cu) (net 2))
 (segment (start 138.136897 95.853517) (end 138.136897 94.827466) (width 0.254) (layer F.Cu) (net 2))
 (segment (start 142.855187 94.822667) (end 146.267333 94.822667) (width 0.254) (layer F.Cu) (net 2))
 (segment (start 147.53 94.82) (end 146.27 94.82) (width 0.254) (layer B.Cu) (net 2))
 (via (at 146.27 94.82) (size 0.6096) (drill 0.3048) (layers F.Cu B.Cu) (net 2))
 (segment (start 146.267333 94.822667) (end 146.27 94.82) (width 0.254) (layer F.Cu) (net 2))
 (segment (start 142.855187 94.822667) (end 140.903854 96.774) (width 0.254) (layer F.Cu) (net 2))
 (segment (start 143.67 96.75) (end 143.78 96.64) (width 0.254) (layer B.Cu) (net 3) (status 30))
 (segment (start 149.731841 91.267281) (end 149.65564 91.19108) (width 0.254) (layer B.Cu) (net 3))
 (segment (start 149.731841 92.113099) (end 149.731841 91.267281) (width 0.254) (layer B.Cu) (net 3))
 (segment (start 149.65564 92.1893) (end 149.731841 92.113099) (width 0.254) (layer B.Cu) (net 3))
 (segment (start 149.02064 92.1893) (end 149.65564 92.1893) (width 0.254) (layer B.Cu) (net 3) (status 10))
 (segment (start 149.65564 91.19108) (end 149.02064 91.19108) (width 0.254) (layer B.Cu) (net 3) (status 20))
 (segment (start 149.02064 91.19108) (end 151.27108 91.19108) (width 0.254) (layer B.Cu) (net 3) (status 30))
 (segment (start 151.27108 91.19108) (end 151.52 91.44) (width 0.254) (layer B.Cu) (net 3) (status 30))
 (segment (start 155.0343 92.43996) (end 155 92.40566) (width 0.254) (layer B.Cu) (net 3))
 (segment (start 156.19 92.43996) (end 155.0343 92.43996) (width 0.254) (layer B.Cu) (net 3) (status 10))
 (segment (start 155 92.40566) (end 155 91.94) (width 0.254) (layer B.Cu) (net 3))
 (segment (start 155 91.94) (end 154.74892 91.68892) (width 0.254) (layer B.Cu) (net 3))
 (segment (start 154.74892 91.68892) (end 154.01936 91.68892) (width 0.254) (layer B.Cu) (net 3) (status 20))
 (segment (start 153.414838 91.68892) (end 154.01936 91.68892) (width 0.254) (layer B.Cu) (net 3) (status 20))
 (segment (start 149.02064 91.19108) (end 152.916998 91.19108) (width 0.254) (layer B.Cu) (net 3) (status 10))
 (segment (start 152.916998 91.19108) (end 153.414838 91.68892) (width 0.254) (layer B.Cu) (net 3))
 (segment (start 152.155 92.075) (end 151.52 91.44) (width 0.254) (layer B.Cu) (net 3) (status 20))
 (segment (start 152.155 92.72) (end 152.155 92.075) (width 0.254) (layer B.Cu) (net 3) (status 10))
 (segment (start 143.425199 92) (end 143.425199 92.123841) (width 0.254) (layer B.Cu) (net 3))
 (segment (start 139.835098 92.544529) (end 139.863103 92.572534) (width 0.254) (layer F.Cu) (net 3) (status 30))
 (segment (start 137.023435 92.544529) (end 139.835098 92.544529) (width 0.254) (layer F.Cu) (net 3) (status 30))
 (segment (start 156.19 94.14164) (end 155.94164 94.39) (width 0.254) (layer B.Cu) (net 3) (status 30))
 (segment (start 143.425199 92.123841) (end 143.425199 90.46) (width 0.254) (layer B.Cu) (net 3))
 (segment (start 143.755199 90.13) (end 145.5 90.13) (width 0.254) (layer B.Cu) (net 3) (status 20))
 (segment (start 143.425199 90.46) (end 143.755199 90.13) (width 0.254) (layer B.Cu) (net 3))
 (segment (start 156.19 92.43996) (end 156.19 94.14164) (width 0.254) (layer B.Cu) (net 3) (status 30))
 (segment (start 135.25246 92.1004) (end 133.025468 93.542076) (width 0.254) (layer B.Cu) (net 3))
 (segment (start 137.023435 92.544529) (end 135.25246 92.1004) (width 0.254) (layer B.Cu) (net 3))
 (segment (start 139.863103 92.572534) (end 143.458894 92.572534) (width 0.254) (layer B.Cu) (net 3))
 (segment (start 146.697466 92.572534) (end 146.775199 92.494801) (width 0.254) (layer B.Cu) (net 3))
 (segment (start 148.07892 91.19108) (end 149.02064 91.19108) (width 0.254) (layer B.Cu) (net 3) (status 10))
 (segment (start 146.775199 92.494801) (end 148.07892 91.19108) (width 0.254) (layer B.Cu) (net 3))
 (segment (start 143.458894 92.572534) (end 143.718426 92.572534) (width 0.254) (layer B.Cu) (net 3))
 (segment (start 143.718426 92.572534) (end 146.697466 92.572534) (width 0.254) (layer B.Cu) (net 3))
 (segment (start 143.425199 92.538839) (end 143.458894 92.572534) (width 0.254) (layer B.Cu) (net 3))
 (segment (start 143.425199 92.123841) (end 143.425199 92.279307) (width 0.254) (layer B.Cu) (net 3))
 (segment (start 143.425199 92.279307) (end 143.425199 92.538839) (width 0.254) (layer B.Cu) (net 3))
 (segment (start 143.425199 96.285199) (end 143.78 96.64) (width 0.254) (layer B.Cu) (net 3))
 (segment (start 143.425199 92.538839) (end 143.425199 96.285199) (width 0.254) (layer B.Cu) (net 3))
 (segment (start 162.72256 99.90582) (end 166.43223 94.7547) (width 0.254) (layer F.Cu) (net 3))
 (via (at 166.43223 94.7547) (size 0.6096) (layers F.Cu B.Cu) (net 3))
 (segment (start 166.43223 94.7547) (end 167.220374 93.433533) (width 0.254) (layer B.Cu) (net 3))
 (segment (start 156.007223 95.259493) (end 156.018969 95.259493) (width 0.254) (layer B.Cu) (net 3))
 (segment (start 159.211052 97.36) (end 157.110545 95.259493) (width 0.254) (layer F.Cu) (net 3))
 (segment (start 156.881073 95.259493) (end 156.450021 95.259493) (width 0.254) (layer F.Cu) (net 3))
 (segment (start 157.110545 95.259493) (end 156.881073 95.259493) (width 0.254) (layer F.Cu) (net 3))
 (segment (start 155.94164 94.39) (end 155.94164 95.19391) (width 0.254) (layer B.Cu) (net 3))
 (segment (start 156.018969 95.259493) (end 156.450021 95.259493) (width 0.254) (layer B.Cu) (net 3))
 (via (at 156.450021 95.259493) (size 0.6096) (drill 0.3048) (layers F.Cu B.Cu) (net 3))
 (segment (start 155.94164 95.19391) (end 156.007223 95.259493) (width 0.254) (layer B.Cu) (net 3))
 (segment (start 159.211052 97.36) (end 162.72256 99.90582) (width 0.254) (layer F.Cu) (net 3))
 (segment (start 158.11 92.25) (end 158.11 93.03) (width 0.254) (layer B.Cu) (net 8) (status 10))
 (segment (start 157.63836 93.50164) (end 157.63836 94.39) (width 0.254) (layer B.Cu) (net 8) (status 20))
 (segment (start 158.11 93.03) (end 157.63836 93.50164) (width 0.254) (layer B.Cu) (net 8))
 (segment (start 157.63836 94.39) (end 157.7 94.32836) (width 0.254) (layer B.Cu) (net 8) (status 30))
 (segment (start 153.27006 93.93936) (end 153.903266 93.93936) (width 0.254) (layer B.Cu) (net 12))
 (segment (start 153.96399 94.37399) (end 153.96399 94.000084) (width 0.254) (layer F.Cu) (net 12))
 (via (at 153.96399 94.000084) (size 0.6096) (drill 0.3048) (layers F.Cu B.Cu) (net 12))
 (segment (start 155.16 95.57) (end 153.96399 94.37399) (width 0.254) (layer F.Cu) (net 12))
 (segment (start 153.903266 93.93936) (end 153.96399 94.000084) (width 0.254) (layer B.Cu) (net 12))
 (segment (start 151.208948 95.3) (end 151.98791 95.3) (width 0.254) (layer F.Cu) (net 12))
 (segment (start 152.208429 95.520519) (end 152.639481 95.520519) (width 0.254) (layer F.Cu) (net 12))
 (segment (start 151.98791 95.3) (end 152.208429 95.520519) (width 0.254) (layer F.Cu) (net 12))
 (via (at 152.639481 95.520519) (size 0.6096) (drill 0.3048) (layers F.Cu B.Cu) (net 12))
 (segment (start 147.66 95.3) (end 151.208948 95.3) (width 0.254) (layer F.Cu) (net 12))
 (segment (start 146.32 96.64) (end 147.66 95.3) (width 0.254) (layer F.Cu) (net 12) (status 10))
 (via (at 155.16 95.57) (size 0.6096) (drill 0.3048) (layers F.Cu B.Cu) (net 12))
 (segment (start 154.89 95.3) (end 155.16 95.57) (width 0.254) (layer B.Cu) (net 12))
 (segment (start 152.86 95.3) (end 154.89 95.3) (width 0.254) (layer B.Cu) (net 12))
 (segment (start 152.639481 95.520519) (end 152.86 95.3) (width 0.254) (layer B.Cu) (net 12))
 (segment (start 157.2084 92.56996) (end 157.27 92.50836) (width 0.254) (layer F.Cu) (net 13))
 (segment (start 155.81502 95.97502) (end 155.81502 94.00795) (width 0.254) (layer F.Cu) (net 13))
 (segment (start 156.48 96.64) (end 155.81502 95.97502) (width 0.254) (layer F.Cu) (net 13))
 (segment (start 156.2733 92.23996) (end 156.34 92.30666) (width 0.254) (layer F.Cu) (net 13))
 (segment (start 155.27 92.23996) (end 156.2733 92.23996) (width 0.254) (layer F.Cu) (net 13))
 (segment (start 156.46609 92.50836) (end 157.27 92.50836) (width 0.254) (layer F.Cu) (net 13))
 (segment (start 156.34 92.38227) (end 156.46609 92.50836) (width 0.254) (layer F.Cu) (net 13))
 (segment (start 156.34 92.30666) (end 156.34 92.38227) (width 0.254) (layer F.Cu) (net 13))
 (segment (start 155.27 93.46293) (end 155.27 92.23996) (width 0.254) (layer F.Cu) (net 13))
 (segment (start 155.81502 94.00795) (end 155.27 93.46293) (width 0.254) (layer F.Cu) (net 13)))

